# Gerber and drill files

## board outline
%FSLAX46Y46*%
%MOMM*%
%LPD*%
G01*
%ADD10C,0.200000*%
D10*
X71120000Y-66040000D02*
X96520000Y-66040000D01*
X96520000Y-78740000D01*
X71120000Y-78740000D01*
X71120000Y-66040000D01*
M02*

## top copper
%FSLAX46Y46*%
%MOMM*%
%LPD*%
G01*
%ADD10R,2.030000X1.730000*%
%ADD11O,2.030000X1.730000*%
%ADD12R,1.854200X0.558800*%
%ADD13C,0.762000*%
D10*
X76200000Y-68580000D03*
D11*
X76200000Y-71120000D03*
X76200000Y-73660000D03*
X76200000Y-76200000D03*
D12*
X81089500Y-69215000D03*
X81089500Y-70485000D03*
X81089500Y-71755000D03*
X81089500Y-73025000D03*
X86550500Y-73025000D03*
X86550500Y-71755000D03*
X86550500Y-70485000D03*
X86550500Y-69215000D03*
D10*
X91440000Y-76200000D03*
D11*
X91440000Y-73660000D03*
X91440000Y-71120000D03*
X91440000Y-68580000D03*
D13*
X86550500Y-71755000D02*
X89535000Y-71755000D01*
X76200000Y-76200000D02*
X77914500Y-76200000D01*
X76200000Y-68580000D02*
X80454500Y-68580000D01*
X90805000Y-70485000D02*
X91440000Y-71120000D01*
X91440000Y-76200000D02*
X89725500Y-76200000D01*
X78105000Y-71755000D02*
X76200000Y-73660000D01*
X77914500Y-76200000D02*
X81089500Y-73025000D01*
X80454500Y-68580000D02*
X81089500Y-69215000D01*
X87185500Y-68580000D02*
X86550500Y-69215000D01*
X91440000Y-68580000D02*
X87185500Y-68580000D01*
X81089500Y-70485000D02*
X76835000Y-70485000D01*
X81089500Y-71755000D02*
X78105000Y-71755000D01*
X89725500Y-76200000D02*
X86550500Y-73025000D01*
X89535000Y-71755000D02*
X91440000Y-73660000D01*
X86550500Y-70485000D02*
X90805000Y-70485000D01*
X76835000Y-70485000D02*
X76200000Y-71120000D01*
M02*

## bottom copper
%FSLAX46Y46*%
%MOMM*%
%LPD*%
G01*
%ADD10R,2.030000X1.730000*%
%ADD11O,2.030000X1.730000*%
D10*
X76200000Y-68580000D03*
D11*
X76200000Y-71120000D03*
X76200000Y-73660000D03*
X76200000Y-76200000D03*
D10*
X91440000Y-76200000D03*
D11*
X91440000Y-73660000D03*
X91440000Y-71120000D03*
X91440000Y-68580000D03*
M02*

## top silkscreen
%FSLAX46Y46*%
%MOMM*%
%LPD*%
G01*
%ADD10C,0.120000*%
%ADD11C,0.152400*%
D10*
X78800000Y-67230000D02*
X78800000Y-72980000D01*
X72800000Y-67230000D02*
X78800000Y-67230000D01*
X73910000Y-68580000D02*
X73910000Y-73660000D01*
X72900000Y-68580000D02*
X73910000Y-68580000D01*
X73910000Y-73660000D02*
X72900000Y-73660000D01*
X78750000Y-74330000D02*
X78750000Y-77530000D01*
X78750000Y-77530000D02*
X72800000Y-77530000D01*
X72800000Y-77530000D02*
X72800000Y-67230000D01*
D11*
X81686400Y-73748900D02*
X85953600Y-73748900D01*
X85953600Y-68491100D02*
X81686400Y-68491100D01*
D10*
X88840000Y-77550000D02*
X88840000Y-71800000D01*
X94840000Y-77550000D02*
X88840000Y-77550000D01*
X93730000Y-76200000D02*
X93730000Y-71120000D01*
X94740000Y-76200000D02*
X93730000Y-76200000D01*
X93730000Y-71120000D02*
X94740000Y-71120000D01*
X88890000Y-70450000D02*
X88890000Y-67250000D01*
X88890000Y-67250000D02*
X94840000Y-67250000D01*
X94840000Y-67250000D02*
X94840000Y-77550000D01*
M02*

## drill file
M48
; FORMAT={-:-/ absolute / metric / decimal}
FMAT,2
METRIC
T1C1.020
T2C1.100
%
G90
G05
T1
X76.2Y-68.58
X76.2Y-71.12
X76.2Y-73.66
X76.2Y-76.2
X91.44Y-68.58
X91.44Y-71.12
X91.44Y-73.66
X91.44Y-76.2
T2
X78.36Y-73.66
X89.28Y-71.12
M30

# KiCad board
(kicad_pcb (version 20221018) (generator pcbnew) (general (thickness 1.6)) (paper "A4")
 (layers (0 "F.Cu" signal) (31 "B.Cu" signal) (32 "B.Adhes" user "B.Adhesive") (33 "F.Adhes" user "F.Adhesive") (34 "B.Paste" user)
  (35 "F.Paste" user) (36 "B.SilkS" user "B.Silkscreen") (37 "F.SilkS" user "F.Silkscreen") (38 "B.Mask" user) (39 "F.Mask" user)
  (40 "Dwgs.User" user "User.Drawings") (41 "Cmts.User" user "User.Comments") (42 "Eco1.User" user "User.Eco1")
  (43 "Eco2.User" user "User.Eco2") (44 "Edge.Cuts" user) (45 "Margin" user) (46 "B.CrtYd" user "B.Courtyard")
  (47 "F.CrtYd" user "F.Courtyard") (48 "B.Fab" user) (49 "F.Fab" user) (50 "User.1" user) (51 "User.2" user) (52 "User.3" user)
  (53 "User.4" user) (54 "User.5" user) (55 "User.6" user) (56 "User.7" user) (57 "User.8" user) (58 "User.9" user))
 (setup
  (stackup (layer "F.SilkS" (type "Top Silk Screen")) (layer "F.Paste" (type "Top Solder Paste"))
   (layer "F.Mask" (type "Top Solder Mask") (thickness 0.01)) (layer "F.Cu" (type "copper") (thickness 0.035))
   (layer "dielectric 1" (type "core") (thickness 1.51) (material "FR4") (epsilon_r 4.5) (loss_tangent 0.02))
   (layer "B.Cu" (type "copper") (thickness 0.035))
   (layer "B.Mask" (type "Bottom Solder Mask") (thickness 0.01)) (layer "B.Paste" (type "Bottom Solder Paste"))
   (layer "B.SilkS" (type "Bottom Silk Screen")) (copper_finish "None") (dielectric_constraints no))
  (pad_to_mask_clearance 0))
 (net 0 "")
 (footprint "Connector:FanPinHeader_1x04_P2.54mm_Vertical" (layer "F.Cu") (at 76.2 68.58 -90)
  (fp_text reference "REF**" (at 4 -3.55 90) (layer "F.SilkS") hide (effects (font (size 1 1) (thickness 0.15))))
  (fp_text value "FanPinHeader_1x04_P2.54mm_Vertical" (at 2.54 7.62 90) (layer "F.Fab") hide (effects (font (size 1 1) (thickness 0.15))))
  (fp_line (start -1.35 -2.6) (end 4.4 -2.6) (stroke (width 0.12) (type solid)) (layer "F.SilkS"))
  (fp_line (start -1.35 3.4) (end -1.35 -2.6) (stroke (width 0.12) (type solid)) (layer "F.SilkS"))
  (fp_line (start 0 2.29) (end 5.08 2.29) (stroke (width 0.12) (type solid)) (layer "F.SilkS"))
  (fp_line (start 0 3.3) (end 0 2.29) (stroke (width 0.12) (type solid)) (layer "F.SilkS"))
  (fp_line (start 5.08 2.29) (end 5.08 3.3) (stroke (width 0.12) (type solid)) (layer "F.SilkS"))
  (fp_line (start 5.75 -2.55) (end 8.95 -2.55) (stroke (width 0.12) (type solid)) (layer "F.SilkS"))
  (fp_line (start 8.95 -2.55) (end 8.95 3.4) (stroke (width 0.12) (type solid)) (layer "F.SilkS"))
  (fp_line (start 8.95 3.4) (end -1.35 3.4) (stroke (width 0.12) (type solid)) (layer "F.SilkS"))
  (pad "" np_thru_hole circle (at 5.08 -2.16) (size 1.1 1.1) (drill 1.1) (layers "*.Cu" "*.Mask"))
  (pad "1" thru_hole rect (at 0 0) (size 2.03 1.73) (drill 1.02) (layers "*.Cu" "*.Mask"))
  (pad "2" thru_hole oval (at 2.54 0) (size 2.03 1.73) (drill 1.02) (layers "*.Cu" "*.Mask"))
  (pad "3" thru_hole oval (at 5.08 0) (size 2.03 1.73) (drill 1.02) (layers "*.Cu" "*.Mask"))
  (pad "4" thru_hole oval (at 7.62 0) (size 2.03 1.73) (drill 1.02) (layers "*.Cu" "*.Mask")))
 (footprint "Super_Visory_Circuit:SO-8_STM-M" (layer "F.Cu") (at 83.82 71.12)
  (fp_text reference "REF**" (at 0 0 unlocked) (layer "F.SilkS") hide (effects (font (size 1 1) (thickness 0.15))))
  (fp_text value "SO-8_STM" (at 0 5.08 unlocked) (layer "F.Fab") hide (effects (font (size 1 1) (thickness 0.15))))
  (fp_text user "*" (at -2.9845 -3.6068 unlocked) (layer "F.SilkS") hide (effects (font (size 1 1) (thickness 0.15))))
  (fp_line (start -2.1336 2.6289) (end 2.1336 2.6289) (stroke (width 0.1524) (type solid)) (layer "F.SilkS"))
  (fp_line (start 2.1336 -2.6289) (end -2.1336 -2.6289) (stroke (width 0.1524) (type solid)) (layer "F.SilkS"))
  (pad "1" smd rect (at -2.7305 -1.905) (size 1.8542 0.5588) (layers "F.Cu" "F.Paste" "F.Mask"))
  (pad "2" smd rect (at -2.7305 -0.635) (size 1.8542 0.5588) (layers "F.Cu" "F.Paste" "F.Mask"))
  (pad "3" smd rect (at -2.7305 0.635) (size 1.8542 0.5588) (layers "F.Cu" "F.Paste" "F.Mask"))
  (pad "4" smd rect (at -2.7305 1.905) (size 1.8542 0.5588) (layers "F.Cu" "F.Paste" "F.Mask"))
  (pad "5" smd rect (at 2.7305 1.905) (size 1.8542 0.5588) (layers "F.Cu" "F.Paste" "F.Mask"))
  (pad "6" smd rect (at 2.7305 0.635) (size 1.8542 0.5588) (layers "F.Cu" "F.Paste" "F.Mask"))
  (pad "7" smd rect (at 2.7305 -0.635) (size 1.8542 0.5588) (layers "F.Cu" "F.Paste" "F.Mask"))
  (pad "8" smd rect (at 2.7305 -1.905) (size 1.8542 0.5588) (layers "F.Cu" "F.Paste" "F.Mask")))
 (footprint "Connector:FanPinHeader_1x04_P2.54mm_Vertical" (layer "F.Cu") (at 91.44 76.2 90)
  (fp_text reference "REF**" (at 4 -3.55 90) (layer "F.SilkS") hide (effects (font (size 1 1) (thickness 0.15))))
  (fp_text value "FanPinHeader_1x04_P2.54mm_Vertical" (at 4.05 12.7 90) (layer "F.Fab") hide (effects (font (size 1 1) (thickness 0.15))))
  (fp_line (start -1.35 -2.6) (end 4.4 -2.6) (stroke (width 0.12) (type solid)) (layer "F.SilkS"))
  (fp_line (start -1.35 3.4) (end -1.35 -2.6) (stroke (width 0.12) (type solid)) (layer "F.SilkS"))
  (fp_line (start 0 2.29) (end 5.08 2.29) (stroke (width 0.12) (type solid)) (layer "F.SilkS"))
  (fp_line (start 0 3.3) (end 0 2.29) (stroke (width 0.12) (type solid)) (layer "F.SilkS"))
  (fp_line (start 5.08 2.29) (end 5.08 3.3) (stroke (width 0.12) (type solid)) (layer "F.SilkS"))
  (fp_line (start 5.75 -2.55) (end 8.95 -2.55) (stroke (width 0.12) (type solid)) (layer "F.SilkS"))
  (fp_line (start 8.95 -2.55) (end 8.95 3.4) (stroke (width 0.12) (type solid)) (layer "F.SilkS"))
  (fp_line (start 8.95 3.4) (end -1.35 3.4) (stroke (width 0.12) (type solid)) (layer "F.SilkS"))
  (pad "" np_thru_hole circle (at 5.08 -2.16 180) (size 1.1 1.1) (drill 1.1) (layers "*.Cu" "*.Mask"))
  (pad "1" thru_hole rect (at 0 0 180) (size 2.03 1.73) (drill 1.02) (layers "*.Cu" "*.Mask"))
  (pad "2" thru_hole oval (at 2.54 0 180) (size 2.03 1.73) (drill 1.02) (layers "*.Cu" "*.Mask"))
  (pad "3" thru_hole oval (at 5.08 0 180) (size 2.03 1.73) (drill 1.02) (layers "*.Cu" "*.Mask"))
  (pad "4" thru_hole oval (at 7.62 0 180) (size 2.03 1.73) (drill 1.02) (layers "*.Cu" "*.Mask")))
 (gr_rect (start 71.12 66.04) (end 96.52 78.74) (stroke (width 0.2) (type default)) (fill none) (layer "Edge.Cuts"))
 (segment (start 86.5505 71.755) (end 89.535 71.755) (width 0.762) (layer "F.Cu") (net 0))
 (segment (start 76.2 76.2) (end 77.9145 76.2) (width 0.762) (layer "F.Cu") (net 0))
 (segment (start 76.2 68.58) (end 80.4545 68.58) (width 0.762) (layer "F.Cu") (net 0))
 (segment (start 90.805 70.485) (end 91.44 71.12) (width 0.762) (layer "F.Cu") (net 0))
 (segment (start 91.44 76.2) (end 89.7255 76.2) (width 0.762) (layer "F.Cu") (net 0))
 (segment (start 78.105 71.755) (end 76.2 73.66) (width 0.762) (layer "F.Cu") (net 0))
 (segment (start 77.9145 76.2) (end 81.0895 73.025) (width 0.762) (layer "F.Cu") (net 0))
 (segment (start 80.4545 68.58) (end 81.0895 69.215) (width 0.762) (layer "F.Cu") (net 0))
 (segment (start 87.1855 68.58) (end 86.5505 69.215) (width 0.762) (layer "F.Cu") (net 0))
 (segment (start 91.44 68.58) (end 87.1855 68.58) (width 0.762) (layer "F.Cu") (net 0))
 (segment (start 81.0895 70.485) (end 76.835 70.485) (width 0.762) (layer "F.Cu") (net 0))
 (segment (start 81.0895 71.755) (end 78.105 71.755) (width 0.762) (layer "F.Cu") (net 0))
 (segment (start 89.7255 76.2) (end 86.5505 73.025) (width 0.762) (layer "F.Cu") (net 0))
 (segment (start 89.535 71.755) (end 91.44 73.66) (width 0.762) (layer "F.Cu") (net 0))
 (segment (start 86.5505 70.485) (end 90.805 70.485) (width 0.762) (layer "F.Cu") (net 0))
 (segment (start 76.835 70.485) (end 76.2 71.12) (width 0.762) (layer "F.Cu") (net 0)))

